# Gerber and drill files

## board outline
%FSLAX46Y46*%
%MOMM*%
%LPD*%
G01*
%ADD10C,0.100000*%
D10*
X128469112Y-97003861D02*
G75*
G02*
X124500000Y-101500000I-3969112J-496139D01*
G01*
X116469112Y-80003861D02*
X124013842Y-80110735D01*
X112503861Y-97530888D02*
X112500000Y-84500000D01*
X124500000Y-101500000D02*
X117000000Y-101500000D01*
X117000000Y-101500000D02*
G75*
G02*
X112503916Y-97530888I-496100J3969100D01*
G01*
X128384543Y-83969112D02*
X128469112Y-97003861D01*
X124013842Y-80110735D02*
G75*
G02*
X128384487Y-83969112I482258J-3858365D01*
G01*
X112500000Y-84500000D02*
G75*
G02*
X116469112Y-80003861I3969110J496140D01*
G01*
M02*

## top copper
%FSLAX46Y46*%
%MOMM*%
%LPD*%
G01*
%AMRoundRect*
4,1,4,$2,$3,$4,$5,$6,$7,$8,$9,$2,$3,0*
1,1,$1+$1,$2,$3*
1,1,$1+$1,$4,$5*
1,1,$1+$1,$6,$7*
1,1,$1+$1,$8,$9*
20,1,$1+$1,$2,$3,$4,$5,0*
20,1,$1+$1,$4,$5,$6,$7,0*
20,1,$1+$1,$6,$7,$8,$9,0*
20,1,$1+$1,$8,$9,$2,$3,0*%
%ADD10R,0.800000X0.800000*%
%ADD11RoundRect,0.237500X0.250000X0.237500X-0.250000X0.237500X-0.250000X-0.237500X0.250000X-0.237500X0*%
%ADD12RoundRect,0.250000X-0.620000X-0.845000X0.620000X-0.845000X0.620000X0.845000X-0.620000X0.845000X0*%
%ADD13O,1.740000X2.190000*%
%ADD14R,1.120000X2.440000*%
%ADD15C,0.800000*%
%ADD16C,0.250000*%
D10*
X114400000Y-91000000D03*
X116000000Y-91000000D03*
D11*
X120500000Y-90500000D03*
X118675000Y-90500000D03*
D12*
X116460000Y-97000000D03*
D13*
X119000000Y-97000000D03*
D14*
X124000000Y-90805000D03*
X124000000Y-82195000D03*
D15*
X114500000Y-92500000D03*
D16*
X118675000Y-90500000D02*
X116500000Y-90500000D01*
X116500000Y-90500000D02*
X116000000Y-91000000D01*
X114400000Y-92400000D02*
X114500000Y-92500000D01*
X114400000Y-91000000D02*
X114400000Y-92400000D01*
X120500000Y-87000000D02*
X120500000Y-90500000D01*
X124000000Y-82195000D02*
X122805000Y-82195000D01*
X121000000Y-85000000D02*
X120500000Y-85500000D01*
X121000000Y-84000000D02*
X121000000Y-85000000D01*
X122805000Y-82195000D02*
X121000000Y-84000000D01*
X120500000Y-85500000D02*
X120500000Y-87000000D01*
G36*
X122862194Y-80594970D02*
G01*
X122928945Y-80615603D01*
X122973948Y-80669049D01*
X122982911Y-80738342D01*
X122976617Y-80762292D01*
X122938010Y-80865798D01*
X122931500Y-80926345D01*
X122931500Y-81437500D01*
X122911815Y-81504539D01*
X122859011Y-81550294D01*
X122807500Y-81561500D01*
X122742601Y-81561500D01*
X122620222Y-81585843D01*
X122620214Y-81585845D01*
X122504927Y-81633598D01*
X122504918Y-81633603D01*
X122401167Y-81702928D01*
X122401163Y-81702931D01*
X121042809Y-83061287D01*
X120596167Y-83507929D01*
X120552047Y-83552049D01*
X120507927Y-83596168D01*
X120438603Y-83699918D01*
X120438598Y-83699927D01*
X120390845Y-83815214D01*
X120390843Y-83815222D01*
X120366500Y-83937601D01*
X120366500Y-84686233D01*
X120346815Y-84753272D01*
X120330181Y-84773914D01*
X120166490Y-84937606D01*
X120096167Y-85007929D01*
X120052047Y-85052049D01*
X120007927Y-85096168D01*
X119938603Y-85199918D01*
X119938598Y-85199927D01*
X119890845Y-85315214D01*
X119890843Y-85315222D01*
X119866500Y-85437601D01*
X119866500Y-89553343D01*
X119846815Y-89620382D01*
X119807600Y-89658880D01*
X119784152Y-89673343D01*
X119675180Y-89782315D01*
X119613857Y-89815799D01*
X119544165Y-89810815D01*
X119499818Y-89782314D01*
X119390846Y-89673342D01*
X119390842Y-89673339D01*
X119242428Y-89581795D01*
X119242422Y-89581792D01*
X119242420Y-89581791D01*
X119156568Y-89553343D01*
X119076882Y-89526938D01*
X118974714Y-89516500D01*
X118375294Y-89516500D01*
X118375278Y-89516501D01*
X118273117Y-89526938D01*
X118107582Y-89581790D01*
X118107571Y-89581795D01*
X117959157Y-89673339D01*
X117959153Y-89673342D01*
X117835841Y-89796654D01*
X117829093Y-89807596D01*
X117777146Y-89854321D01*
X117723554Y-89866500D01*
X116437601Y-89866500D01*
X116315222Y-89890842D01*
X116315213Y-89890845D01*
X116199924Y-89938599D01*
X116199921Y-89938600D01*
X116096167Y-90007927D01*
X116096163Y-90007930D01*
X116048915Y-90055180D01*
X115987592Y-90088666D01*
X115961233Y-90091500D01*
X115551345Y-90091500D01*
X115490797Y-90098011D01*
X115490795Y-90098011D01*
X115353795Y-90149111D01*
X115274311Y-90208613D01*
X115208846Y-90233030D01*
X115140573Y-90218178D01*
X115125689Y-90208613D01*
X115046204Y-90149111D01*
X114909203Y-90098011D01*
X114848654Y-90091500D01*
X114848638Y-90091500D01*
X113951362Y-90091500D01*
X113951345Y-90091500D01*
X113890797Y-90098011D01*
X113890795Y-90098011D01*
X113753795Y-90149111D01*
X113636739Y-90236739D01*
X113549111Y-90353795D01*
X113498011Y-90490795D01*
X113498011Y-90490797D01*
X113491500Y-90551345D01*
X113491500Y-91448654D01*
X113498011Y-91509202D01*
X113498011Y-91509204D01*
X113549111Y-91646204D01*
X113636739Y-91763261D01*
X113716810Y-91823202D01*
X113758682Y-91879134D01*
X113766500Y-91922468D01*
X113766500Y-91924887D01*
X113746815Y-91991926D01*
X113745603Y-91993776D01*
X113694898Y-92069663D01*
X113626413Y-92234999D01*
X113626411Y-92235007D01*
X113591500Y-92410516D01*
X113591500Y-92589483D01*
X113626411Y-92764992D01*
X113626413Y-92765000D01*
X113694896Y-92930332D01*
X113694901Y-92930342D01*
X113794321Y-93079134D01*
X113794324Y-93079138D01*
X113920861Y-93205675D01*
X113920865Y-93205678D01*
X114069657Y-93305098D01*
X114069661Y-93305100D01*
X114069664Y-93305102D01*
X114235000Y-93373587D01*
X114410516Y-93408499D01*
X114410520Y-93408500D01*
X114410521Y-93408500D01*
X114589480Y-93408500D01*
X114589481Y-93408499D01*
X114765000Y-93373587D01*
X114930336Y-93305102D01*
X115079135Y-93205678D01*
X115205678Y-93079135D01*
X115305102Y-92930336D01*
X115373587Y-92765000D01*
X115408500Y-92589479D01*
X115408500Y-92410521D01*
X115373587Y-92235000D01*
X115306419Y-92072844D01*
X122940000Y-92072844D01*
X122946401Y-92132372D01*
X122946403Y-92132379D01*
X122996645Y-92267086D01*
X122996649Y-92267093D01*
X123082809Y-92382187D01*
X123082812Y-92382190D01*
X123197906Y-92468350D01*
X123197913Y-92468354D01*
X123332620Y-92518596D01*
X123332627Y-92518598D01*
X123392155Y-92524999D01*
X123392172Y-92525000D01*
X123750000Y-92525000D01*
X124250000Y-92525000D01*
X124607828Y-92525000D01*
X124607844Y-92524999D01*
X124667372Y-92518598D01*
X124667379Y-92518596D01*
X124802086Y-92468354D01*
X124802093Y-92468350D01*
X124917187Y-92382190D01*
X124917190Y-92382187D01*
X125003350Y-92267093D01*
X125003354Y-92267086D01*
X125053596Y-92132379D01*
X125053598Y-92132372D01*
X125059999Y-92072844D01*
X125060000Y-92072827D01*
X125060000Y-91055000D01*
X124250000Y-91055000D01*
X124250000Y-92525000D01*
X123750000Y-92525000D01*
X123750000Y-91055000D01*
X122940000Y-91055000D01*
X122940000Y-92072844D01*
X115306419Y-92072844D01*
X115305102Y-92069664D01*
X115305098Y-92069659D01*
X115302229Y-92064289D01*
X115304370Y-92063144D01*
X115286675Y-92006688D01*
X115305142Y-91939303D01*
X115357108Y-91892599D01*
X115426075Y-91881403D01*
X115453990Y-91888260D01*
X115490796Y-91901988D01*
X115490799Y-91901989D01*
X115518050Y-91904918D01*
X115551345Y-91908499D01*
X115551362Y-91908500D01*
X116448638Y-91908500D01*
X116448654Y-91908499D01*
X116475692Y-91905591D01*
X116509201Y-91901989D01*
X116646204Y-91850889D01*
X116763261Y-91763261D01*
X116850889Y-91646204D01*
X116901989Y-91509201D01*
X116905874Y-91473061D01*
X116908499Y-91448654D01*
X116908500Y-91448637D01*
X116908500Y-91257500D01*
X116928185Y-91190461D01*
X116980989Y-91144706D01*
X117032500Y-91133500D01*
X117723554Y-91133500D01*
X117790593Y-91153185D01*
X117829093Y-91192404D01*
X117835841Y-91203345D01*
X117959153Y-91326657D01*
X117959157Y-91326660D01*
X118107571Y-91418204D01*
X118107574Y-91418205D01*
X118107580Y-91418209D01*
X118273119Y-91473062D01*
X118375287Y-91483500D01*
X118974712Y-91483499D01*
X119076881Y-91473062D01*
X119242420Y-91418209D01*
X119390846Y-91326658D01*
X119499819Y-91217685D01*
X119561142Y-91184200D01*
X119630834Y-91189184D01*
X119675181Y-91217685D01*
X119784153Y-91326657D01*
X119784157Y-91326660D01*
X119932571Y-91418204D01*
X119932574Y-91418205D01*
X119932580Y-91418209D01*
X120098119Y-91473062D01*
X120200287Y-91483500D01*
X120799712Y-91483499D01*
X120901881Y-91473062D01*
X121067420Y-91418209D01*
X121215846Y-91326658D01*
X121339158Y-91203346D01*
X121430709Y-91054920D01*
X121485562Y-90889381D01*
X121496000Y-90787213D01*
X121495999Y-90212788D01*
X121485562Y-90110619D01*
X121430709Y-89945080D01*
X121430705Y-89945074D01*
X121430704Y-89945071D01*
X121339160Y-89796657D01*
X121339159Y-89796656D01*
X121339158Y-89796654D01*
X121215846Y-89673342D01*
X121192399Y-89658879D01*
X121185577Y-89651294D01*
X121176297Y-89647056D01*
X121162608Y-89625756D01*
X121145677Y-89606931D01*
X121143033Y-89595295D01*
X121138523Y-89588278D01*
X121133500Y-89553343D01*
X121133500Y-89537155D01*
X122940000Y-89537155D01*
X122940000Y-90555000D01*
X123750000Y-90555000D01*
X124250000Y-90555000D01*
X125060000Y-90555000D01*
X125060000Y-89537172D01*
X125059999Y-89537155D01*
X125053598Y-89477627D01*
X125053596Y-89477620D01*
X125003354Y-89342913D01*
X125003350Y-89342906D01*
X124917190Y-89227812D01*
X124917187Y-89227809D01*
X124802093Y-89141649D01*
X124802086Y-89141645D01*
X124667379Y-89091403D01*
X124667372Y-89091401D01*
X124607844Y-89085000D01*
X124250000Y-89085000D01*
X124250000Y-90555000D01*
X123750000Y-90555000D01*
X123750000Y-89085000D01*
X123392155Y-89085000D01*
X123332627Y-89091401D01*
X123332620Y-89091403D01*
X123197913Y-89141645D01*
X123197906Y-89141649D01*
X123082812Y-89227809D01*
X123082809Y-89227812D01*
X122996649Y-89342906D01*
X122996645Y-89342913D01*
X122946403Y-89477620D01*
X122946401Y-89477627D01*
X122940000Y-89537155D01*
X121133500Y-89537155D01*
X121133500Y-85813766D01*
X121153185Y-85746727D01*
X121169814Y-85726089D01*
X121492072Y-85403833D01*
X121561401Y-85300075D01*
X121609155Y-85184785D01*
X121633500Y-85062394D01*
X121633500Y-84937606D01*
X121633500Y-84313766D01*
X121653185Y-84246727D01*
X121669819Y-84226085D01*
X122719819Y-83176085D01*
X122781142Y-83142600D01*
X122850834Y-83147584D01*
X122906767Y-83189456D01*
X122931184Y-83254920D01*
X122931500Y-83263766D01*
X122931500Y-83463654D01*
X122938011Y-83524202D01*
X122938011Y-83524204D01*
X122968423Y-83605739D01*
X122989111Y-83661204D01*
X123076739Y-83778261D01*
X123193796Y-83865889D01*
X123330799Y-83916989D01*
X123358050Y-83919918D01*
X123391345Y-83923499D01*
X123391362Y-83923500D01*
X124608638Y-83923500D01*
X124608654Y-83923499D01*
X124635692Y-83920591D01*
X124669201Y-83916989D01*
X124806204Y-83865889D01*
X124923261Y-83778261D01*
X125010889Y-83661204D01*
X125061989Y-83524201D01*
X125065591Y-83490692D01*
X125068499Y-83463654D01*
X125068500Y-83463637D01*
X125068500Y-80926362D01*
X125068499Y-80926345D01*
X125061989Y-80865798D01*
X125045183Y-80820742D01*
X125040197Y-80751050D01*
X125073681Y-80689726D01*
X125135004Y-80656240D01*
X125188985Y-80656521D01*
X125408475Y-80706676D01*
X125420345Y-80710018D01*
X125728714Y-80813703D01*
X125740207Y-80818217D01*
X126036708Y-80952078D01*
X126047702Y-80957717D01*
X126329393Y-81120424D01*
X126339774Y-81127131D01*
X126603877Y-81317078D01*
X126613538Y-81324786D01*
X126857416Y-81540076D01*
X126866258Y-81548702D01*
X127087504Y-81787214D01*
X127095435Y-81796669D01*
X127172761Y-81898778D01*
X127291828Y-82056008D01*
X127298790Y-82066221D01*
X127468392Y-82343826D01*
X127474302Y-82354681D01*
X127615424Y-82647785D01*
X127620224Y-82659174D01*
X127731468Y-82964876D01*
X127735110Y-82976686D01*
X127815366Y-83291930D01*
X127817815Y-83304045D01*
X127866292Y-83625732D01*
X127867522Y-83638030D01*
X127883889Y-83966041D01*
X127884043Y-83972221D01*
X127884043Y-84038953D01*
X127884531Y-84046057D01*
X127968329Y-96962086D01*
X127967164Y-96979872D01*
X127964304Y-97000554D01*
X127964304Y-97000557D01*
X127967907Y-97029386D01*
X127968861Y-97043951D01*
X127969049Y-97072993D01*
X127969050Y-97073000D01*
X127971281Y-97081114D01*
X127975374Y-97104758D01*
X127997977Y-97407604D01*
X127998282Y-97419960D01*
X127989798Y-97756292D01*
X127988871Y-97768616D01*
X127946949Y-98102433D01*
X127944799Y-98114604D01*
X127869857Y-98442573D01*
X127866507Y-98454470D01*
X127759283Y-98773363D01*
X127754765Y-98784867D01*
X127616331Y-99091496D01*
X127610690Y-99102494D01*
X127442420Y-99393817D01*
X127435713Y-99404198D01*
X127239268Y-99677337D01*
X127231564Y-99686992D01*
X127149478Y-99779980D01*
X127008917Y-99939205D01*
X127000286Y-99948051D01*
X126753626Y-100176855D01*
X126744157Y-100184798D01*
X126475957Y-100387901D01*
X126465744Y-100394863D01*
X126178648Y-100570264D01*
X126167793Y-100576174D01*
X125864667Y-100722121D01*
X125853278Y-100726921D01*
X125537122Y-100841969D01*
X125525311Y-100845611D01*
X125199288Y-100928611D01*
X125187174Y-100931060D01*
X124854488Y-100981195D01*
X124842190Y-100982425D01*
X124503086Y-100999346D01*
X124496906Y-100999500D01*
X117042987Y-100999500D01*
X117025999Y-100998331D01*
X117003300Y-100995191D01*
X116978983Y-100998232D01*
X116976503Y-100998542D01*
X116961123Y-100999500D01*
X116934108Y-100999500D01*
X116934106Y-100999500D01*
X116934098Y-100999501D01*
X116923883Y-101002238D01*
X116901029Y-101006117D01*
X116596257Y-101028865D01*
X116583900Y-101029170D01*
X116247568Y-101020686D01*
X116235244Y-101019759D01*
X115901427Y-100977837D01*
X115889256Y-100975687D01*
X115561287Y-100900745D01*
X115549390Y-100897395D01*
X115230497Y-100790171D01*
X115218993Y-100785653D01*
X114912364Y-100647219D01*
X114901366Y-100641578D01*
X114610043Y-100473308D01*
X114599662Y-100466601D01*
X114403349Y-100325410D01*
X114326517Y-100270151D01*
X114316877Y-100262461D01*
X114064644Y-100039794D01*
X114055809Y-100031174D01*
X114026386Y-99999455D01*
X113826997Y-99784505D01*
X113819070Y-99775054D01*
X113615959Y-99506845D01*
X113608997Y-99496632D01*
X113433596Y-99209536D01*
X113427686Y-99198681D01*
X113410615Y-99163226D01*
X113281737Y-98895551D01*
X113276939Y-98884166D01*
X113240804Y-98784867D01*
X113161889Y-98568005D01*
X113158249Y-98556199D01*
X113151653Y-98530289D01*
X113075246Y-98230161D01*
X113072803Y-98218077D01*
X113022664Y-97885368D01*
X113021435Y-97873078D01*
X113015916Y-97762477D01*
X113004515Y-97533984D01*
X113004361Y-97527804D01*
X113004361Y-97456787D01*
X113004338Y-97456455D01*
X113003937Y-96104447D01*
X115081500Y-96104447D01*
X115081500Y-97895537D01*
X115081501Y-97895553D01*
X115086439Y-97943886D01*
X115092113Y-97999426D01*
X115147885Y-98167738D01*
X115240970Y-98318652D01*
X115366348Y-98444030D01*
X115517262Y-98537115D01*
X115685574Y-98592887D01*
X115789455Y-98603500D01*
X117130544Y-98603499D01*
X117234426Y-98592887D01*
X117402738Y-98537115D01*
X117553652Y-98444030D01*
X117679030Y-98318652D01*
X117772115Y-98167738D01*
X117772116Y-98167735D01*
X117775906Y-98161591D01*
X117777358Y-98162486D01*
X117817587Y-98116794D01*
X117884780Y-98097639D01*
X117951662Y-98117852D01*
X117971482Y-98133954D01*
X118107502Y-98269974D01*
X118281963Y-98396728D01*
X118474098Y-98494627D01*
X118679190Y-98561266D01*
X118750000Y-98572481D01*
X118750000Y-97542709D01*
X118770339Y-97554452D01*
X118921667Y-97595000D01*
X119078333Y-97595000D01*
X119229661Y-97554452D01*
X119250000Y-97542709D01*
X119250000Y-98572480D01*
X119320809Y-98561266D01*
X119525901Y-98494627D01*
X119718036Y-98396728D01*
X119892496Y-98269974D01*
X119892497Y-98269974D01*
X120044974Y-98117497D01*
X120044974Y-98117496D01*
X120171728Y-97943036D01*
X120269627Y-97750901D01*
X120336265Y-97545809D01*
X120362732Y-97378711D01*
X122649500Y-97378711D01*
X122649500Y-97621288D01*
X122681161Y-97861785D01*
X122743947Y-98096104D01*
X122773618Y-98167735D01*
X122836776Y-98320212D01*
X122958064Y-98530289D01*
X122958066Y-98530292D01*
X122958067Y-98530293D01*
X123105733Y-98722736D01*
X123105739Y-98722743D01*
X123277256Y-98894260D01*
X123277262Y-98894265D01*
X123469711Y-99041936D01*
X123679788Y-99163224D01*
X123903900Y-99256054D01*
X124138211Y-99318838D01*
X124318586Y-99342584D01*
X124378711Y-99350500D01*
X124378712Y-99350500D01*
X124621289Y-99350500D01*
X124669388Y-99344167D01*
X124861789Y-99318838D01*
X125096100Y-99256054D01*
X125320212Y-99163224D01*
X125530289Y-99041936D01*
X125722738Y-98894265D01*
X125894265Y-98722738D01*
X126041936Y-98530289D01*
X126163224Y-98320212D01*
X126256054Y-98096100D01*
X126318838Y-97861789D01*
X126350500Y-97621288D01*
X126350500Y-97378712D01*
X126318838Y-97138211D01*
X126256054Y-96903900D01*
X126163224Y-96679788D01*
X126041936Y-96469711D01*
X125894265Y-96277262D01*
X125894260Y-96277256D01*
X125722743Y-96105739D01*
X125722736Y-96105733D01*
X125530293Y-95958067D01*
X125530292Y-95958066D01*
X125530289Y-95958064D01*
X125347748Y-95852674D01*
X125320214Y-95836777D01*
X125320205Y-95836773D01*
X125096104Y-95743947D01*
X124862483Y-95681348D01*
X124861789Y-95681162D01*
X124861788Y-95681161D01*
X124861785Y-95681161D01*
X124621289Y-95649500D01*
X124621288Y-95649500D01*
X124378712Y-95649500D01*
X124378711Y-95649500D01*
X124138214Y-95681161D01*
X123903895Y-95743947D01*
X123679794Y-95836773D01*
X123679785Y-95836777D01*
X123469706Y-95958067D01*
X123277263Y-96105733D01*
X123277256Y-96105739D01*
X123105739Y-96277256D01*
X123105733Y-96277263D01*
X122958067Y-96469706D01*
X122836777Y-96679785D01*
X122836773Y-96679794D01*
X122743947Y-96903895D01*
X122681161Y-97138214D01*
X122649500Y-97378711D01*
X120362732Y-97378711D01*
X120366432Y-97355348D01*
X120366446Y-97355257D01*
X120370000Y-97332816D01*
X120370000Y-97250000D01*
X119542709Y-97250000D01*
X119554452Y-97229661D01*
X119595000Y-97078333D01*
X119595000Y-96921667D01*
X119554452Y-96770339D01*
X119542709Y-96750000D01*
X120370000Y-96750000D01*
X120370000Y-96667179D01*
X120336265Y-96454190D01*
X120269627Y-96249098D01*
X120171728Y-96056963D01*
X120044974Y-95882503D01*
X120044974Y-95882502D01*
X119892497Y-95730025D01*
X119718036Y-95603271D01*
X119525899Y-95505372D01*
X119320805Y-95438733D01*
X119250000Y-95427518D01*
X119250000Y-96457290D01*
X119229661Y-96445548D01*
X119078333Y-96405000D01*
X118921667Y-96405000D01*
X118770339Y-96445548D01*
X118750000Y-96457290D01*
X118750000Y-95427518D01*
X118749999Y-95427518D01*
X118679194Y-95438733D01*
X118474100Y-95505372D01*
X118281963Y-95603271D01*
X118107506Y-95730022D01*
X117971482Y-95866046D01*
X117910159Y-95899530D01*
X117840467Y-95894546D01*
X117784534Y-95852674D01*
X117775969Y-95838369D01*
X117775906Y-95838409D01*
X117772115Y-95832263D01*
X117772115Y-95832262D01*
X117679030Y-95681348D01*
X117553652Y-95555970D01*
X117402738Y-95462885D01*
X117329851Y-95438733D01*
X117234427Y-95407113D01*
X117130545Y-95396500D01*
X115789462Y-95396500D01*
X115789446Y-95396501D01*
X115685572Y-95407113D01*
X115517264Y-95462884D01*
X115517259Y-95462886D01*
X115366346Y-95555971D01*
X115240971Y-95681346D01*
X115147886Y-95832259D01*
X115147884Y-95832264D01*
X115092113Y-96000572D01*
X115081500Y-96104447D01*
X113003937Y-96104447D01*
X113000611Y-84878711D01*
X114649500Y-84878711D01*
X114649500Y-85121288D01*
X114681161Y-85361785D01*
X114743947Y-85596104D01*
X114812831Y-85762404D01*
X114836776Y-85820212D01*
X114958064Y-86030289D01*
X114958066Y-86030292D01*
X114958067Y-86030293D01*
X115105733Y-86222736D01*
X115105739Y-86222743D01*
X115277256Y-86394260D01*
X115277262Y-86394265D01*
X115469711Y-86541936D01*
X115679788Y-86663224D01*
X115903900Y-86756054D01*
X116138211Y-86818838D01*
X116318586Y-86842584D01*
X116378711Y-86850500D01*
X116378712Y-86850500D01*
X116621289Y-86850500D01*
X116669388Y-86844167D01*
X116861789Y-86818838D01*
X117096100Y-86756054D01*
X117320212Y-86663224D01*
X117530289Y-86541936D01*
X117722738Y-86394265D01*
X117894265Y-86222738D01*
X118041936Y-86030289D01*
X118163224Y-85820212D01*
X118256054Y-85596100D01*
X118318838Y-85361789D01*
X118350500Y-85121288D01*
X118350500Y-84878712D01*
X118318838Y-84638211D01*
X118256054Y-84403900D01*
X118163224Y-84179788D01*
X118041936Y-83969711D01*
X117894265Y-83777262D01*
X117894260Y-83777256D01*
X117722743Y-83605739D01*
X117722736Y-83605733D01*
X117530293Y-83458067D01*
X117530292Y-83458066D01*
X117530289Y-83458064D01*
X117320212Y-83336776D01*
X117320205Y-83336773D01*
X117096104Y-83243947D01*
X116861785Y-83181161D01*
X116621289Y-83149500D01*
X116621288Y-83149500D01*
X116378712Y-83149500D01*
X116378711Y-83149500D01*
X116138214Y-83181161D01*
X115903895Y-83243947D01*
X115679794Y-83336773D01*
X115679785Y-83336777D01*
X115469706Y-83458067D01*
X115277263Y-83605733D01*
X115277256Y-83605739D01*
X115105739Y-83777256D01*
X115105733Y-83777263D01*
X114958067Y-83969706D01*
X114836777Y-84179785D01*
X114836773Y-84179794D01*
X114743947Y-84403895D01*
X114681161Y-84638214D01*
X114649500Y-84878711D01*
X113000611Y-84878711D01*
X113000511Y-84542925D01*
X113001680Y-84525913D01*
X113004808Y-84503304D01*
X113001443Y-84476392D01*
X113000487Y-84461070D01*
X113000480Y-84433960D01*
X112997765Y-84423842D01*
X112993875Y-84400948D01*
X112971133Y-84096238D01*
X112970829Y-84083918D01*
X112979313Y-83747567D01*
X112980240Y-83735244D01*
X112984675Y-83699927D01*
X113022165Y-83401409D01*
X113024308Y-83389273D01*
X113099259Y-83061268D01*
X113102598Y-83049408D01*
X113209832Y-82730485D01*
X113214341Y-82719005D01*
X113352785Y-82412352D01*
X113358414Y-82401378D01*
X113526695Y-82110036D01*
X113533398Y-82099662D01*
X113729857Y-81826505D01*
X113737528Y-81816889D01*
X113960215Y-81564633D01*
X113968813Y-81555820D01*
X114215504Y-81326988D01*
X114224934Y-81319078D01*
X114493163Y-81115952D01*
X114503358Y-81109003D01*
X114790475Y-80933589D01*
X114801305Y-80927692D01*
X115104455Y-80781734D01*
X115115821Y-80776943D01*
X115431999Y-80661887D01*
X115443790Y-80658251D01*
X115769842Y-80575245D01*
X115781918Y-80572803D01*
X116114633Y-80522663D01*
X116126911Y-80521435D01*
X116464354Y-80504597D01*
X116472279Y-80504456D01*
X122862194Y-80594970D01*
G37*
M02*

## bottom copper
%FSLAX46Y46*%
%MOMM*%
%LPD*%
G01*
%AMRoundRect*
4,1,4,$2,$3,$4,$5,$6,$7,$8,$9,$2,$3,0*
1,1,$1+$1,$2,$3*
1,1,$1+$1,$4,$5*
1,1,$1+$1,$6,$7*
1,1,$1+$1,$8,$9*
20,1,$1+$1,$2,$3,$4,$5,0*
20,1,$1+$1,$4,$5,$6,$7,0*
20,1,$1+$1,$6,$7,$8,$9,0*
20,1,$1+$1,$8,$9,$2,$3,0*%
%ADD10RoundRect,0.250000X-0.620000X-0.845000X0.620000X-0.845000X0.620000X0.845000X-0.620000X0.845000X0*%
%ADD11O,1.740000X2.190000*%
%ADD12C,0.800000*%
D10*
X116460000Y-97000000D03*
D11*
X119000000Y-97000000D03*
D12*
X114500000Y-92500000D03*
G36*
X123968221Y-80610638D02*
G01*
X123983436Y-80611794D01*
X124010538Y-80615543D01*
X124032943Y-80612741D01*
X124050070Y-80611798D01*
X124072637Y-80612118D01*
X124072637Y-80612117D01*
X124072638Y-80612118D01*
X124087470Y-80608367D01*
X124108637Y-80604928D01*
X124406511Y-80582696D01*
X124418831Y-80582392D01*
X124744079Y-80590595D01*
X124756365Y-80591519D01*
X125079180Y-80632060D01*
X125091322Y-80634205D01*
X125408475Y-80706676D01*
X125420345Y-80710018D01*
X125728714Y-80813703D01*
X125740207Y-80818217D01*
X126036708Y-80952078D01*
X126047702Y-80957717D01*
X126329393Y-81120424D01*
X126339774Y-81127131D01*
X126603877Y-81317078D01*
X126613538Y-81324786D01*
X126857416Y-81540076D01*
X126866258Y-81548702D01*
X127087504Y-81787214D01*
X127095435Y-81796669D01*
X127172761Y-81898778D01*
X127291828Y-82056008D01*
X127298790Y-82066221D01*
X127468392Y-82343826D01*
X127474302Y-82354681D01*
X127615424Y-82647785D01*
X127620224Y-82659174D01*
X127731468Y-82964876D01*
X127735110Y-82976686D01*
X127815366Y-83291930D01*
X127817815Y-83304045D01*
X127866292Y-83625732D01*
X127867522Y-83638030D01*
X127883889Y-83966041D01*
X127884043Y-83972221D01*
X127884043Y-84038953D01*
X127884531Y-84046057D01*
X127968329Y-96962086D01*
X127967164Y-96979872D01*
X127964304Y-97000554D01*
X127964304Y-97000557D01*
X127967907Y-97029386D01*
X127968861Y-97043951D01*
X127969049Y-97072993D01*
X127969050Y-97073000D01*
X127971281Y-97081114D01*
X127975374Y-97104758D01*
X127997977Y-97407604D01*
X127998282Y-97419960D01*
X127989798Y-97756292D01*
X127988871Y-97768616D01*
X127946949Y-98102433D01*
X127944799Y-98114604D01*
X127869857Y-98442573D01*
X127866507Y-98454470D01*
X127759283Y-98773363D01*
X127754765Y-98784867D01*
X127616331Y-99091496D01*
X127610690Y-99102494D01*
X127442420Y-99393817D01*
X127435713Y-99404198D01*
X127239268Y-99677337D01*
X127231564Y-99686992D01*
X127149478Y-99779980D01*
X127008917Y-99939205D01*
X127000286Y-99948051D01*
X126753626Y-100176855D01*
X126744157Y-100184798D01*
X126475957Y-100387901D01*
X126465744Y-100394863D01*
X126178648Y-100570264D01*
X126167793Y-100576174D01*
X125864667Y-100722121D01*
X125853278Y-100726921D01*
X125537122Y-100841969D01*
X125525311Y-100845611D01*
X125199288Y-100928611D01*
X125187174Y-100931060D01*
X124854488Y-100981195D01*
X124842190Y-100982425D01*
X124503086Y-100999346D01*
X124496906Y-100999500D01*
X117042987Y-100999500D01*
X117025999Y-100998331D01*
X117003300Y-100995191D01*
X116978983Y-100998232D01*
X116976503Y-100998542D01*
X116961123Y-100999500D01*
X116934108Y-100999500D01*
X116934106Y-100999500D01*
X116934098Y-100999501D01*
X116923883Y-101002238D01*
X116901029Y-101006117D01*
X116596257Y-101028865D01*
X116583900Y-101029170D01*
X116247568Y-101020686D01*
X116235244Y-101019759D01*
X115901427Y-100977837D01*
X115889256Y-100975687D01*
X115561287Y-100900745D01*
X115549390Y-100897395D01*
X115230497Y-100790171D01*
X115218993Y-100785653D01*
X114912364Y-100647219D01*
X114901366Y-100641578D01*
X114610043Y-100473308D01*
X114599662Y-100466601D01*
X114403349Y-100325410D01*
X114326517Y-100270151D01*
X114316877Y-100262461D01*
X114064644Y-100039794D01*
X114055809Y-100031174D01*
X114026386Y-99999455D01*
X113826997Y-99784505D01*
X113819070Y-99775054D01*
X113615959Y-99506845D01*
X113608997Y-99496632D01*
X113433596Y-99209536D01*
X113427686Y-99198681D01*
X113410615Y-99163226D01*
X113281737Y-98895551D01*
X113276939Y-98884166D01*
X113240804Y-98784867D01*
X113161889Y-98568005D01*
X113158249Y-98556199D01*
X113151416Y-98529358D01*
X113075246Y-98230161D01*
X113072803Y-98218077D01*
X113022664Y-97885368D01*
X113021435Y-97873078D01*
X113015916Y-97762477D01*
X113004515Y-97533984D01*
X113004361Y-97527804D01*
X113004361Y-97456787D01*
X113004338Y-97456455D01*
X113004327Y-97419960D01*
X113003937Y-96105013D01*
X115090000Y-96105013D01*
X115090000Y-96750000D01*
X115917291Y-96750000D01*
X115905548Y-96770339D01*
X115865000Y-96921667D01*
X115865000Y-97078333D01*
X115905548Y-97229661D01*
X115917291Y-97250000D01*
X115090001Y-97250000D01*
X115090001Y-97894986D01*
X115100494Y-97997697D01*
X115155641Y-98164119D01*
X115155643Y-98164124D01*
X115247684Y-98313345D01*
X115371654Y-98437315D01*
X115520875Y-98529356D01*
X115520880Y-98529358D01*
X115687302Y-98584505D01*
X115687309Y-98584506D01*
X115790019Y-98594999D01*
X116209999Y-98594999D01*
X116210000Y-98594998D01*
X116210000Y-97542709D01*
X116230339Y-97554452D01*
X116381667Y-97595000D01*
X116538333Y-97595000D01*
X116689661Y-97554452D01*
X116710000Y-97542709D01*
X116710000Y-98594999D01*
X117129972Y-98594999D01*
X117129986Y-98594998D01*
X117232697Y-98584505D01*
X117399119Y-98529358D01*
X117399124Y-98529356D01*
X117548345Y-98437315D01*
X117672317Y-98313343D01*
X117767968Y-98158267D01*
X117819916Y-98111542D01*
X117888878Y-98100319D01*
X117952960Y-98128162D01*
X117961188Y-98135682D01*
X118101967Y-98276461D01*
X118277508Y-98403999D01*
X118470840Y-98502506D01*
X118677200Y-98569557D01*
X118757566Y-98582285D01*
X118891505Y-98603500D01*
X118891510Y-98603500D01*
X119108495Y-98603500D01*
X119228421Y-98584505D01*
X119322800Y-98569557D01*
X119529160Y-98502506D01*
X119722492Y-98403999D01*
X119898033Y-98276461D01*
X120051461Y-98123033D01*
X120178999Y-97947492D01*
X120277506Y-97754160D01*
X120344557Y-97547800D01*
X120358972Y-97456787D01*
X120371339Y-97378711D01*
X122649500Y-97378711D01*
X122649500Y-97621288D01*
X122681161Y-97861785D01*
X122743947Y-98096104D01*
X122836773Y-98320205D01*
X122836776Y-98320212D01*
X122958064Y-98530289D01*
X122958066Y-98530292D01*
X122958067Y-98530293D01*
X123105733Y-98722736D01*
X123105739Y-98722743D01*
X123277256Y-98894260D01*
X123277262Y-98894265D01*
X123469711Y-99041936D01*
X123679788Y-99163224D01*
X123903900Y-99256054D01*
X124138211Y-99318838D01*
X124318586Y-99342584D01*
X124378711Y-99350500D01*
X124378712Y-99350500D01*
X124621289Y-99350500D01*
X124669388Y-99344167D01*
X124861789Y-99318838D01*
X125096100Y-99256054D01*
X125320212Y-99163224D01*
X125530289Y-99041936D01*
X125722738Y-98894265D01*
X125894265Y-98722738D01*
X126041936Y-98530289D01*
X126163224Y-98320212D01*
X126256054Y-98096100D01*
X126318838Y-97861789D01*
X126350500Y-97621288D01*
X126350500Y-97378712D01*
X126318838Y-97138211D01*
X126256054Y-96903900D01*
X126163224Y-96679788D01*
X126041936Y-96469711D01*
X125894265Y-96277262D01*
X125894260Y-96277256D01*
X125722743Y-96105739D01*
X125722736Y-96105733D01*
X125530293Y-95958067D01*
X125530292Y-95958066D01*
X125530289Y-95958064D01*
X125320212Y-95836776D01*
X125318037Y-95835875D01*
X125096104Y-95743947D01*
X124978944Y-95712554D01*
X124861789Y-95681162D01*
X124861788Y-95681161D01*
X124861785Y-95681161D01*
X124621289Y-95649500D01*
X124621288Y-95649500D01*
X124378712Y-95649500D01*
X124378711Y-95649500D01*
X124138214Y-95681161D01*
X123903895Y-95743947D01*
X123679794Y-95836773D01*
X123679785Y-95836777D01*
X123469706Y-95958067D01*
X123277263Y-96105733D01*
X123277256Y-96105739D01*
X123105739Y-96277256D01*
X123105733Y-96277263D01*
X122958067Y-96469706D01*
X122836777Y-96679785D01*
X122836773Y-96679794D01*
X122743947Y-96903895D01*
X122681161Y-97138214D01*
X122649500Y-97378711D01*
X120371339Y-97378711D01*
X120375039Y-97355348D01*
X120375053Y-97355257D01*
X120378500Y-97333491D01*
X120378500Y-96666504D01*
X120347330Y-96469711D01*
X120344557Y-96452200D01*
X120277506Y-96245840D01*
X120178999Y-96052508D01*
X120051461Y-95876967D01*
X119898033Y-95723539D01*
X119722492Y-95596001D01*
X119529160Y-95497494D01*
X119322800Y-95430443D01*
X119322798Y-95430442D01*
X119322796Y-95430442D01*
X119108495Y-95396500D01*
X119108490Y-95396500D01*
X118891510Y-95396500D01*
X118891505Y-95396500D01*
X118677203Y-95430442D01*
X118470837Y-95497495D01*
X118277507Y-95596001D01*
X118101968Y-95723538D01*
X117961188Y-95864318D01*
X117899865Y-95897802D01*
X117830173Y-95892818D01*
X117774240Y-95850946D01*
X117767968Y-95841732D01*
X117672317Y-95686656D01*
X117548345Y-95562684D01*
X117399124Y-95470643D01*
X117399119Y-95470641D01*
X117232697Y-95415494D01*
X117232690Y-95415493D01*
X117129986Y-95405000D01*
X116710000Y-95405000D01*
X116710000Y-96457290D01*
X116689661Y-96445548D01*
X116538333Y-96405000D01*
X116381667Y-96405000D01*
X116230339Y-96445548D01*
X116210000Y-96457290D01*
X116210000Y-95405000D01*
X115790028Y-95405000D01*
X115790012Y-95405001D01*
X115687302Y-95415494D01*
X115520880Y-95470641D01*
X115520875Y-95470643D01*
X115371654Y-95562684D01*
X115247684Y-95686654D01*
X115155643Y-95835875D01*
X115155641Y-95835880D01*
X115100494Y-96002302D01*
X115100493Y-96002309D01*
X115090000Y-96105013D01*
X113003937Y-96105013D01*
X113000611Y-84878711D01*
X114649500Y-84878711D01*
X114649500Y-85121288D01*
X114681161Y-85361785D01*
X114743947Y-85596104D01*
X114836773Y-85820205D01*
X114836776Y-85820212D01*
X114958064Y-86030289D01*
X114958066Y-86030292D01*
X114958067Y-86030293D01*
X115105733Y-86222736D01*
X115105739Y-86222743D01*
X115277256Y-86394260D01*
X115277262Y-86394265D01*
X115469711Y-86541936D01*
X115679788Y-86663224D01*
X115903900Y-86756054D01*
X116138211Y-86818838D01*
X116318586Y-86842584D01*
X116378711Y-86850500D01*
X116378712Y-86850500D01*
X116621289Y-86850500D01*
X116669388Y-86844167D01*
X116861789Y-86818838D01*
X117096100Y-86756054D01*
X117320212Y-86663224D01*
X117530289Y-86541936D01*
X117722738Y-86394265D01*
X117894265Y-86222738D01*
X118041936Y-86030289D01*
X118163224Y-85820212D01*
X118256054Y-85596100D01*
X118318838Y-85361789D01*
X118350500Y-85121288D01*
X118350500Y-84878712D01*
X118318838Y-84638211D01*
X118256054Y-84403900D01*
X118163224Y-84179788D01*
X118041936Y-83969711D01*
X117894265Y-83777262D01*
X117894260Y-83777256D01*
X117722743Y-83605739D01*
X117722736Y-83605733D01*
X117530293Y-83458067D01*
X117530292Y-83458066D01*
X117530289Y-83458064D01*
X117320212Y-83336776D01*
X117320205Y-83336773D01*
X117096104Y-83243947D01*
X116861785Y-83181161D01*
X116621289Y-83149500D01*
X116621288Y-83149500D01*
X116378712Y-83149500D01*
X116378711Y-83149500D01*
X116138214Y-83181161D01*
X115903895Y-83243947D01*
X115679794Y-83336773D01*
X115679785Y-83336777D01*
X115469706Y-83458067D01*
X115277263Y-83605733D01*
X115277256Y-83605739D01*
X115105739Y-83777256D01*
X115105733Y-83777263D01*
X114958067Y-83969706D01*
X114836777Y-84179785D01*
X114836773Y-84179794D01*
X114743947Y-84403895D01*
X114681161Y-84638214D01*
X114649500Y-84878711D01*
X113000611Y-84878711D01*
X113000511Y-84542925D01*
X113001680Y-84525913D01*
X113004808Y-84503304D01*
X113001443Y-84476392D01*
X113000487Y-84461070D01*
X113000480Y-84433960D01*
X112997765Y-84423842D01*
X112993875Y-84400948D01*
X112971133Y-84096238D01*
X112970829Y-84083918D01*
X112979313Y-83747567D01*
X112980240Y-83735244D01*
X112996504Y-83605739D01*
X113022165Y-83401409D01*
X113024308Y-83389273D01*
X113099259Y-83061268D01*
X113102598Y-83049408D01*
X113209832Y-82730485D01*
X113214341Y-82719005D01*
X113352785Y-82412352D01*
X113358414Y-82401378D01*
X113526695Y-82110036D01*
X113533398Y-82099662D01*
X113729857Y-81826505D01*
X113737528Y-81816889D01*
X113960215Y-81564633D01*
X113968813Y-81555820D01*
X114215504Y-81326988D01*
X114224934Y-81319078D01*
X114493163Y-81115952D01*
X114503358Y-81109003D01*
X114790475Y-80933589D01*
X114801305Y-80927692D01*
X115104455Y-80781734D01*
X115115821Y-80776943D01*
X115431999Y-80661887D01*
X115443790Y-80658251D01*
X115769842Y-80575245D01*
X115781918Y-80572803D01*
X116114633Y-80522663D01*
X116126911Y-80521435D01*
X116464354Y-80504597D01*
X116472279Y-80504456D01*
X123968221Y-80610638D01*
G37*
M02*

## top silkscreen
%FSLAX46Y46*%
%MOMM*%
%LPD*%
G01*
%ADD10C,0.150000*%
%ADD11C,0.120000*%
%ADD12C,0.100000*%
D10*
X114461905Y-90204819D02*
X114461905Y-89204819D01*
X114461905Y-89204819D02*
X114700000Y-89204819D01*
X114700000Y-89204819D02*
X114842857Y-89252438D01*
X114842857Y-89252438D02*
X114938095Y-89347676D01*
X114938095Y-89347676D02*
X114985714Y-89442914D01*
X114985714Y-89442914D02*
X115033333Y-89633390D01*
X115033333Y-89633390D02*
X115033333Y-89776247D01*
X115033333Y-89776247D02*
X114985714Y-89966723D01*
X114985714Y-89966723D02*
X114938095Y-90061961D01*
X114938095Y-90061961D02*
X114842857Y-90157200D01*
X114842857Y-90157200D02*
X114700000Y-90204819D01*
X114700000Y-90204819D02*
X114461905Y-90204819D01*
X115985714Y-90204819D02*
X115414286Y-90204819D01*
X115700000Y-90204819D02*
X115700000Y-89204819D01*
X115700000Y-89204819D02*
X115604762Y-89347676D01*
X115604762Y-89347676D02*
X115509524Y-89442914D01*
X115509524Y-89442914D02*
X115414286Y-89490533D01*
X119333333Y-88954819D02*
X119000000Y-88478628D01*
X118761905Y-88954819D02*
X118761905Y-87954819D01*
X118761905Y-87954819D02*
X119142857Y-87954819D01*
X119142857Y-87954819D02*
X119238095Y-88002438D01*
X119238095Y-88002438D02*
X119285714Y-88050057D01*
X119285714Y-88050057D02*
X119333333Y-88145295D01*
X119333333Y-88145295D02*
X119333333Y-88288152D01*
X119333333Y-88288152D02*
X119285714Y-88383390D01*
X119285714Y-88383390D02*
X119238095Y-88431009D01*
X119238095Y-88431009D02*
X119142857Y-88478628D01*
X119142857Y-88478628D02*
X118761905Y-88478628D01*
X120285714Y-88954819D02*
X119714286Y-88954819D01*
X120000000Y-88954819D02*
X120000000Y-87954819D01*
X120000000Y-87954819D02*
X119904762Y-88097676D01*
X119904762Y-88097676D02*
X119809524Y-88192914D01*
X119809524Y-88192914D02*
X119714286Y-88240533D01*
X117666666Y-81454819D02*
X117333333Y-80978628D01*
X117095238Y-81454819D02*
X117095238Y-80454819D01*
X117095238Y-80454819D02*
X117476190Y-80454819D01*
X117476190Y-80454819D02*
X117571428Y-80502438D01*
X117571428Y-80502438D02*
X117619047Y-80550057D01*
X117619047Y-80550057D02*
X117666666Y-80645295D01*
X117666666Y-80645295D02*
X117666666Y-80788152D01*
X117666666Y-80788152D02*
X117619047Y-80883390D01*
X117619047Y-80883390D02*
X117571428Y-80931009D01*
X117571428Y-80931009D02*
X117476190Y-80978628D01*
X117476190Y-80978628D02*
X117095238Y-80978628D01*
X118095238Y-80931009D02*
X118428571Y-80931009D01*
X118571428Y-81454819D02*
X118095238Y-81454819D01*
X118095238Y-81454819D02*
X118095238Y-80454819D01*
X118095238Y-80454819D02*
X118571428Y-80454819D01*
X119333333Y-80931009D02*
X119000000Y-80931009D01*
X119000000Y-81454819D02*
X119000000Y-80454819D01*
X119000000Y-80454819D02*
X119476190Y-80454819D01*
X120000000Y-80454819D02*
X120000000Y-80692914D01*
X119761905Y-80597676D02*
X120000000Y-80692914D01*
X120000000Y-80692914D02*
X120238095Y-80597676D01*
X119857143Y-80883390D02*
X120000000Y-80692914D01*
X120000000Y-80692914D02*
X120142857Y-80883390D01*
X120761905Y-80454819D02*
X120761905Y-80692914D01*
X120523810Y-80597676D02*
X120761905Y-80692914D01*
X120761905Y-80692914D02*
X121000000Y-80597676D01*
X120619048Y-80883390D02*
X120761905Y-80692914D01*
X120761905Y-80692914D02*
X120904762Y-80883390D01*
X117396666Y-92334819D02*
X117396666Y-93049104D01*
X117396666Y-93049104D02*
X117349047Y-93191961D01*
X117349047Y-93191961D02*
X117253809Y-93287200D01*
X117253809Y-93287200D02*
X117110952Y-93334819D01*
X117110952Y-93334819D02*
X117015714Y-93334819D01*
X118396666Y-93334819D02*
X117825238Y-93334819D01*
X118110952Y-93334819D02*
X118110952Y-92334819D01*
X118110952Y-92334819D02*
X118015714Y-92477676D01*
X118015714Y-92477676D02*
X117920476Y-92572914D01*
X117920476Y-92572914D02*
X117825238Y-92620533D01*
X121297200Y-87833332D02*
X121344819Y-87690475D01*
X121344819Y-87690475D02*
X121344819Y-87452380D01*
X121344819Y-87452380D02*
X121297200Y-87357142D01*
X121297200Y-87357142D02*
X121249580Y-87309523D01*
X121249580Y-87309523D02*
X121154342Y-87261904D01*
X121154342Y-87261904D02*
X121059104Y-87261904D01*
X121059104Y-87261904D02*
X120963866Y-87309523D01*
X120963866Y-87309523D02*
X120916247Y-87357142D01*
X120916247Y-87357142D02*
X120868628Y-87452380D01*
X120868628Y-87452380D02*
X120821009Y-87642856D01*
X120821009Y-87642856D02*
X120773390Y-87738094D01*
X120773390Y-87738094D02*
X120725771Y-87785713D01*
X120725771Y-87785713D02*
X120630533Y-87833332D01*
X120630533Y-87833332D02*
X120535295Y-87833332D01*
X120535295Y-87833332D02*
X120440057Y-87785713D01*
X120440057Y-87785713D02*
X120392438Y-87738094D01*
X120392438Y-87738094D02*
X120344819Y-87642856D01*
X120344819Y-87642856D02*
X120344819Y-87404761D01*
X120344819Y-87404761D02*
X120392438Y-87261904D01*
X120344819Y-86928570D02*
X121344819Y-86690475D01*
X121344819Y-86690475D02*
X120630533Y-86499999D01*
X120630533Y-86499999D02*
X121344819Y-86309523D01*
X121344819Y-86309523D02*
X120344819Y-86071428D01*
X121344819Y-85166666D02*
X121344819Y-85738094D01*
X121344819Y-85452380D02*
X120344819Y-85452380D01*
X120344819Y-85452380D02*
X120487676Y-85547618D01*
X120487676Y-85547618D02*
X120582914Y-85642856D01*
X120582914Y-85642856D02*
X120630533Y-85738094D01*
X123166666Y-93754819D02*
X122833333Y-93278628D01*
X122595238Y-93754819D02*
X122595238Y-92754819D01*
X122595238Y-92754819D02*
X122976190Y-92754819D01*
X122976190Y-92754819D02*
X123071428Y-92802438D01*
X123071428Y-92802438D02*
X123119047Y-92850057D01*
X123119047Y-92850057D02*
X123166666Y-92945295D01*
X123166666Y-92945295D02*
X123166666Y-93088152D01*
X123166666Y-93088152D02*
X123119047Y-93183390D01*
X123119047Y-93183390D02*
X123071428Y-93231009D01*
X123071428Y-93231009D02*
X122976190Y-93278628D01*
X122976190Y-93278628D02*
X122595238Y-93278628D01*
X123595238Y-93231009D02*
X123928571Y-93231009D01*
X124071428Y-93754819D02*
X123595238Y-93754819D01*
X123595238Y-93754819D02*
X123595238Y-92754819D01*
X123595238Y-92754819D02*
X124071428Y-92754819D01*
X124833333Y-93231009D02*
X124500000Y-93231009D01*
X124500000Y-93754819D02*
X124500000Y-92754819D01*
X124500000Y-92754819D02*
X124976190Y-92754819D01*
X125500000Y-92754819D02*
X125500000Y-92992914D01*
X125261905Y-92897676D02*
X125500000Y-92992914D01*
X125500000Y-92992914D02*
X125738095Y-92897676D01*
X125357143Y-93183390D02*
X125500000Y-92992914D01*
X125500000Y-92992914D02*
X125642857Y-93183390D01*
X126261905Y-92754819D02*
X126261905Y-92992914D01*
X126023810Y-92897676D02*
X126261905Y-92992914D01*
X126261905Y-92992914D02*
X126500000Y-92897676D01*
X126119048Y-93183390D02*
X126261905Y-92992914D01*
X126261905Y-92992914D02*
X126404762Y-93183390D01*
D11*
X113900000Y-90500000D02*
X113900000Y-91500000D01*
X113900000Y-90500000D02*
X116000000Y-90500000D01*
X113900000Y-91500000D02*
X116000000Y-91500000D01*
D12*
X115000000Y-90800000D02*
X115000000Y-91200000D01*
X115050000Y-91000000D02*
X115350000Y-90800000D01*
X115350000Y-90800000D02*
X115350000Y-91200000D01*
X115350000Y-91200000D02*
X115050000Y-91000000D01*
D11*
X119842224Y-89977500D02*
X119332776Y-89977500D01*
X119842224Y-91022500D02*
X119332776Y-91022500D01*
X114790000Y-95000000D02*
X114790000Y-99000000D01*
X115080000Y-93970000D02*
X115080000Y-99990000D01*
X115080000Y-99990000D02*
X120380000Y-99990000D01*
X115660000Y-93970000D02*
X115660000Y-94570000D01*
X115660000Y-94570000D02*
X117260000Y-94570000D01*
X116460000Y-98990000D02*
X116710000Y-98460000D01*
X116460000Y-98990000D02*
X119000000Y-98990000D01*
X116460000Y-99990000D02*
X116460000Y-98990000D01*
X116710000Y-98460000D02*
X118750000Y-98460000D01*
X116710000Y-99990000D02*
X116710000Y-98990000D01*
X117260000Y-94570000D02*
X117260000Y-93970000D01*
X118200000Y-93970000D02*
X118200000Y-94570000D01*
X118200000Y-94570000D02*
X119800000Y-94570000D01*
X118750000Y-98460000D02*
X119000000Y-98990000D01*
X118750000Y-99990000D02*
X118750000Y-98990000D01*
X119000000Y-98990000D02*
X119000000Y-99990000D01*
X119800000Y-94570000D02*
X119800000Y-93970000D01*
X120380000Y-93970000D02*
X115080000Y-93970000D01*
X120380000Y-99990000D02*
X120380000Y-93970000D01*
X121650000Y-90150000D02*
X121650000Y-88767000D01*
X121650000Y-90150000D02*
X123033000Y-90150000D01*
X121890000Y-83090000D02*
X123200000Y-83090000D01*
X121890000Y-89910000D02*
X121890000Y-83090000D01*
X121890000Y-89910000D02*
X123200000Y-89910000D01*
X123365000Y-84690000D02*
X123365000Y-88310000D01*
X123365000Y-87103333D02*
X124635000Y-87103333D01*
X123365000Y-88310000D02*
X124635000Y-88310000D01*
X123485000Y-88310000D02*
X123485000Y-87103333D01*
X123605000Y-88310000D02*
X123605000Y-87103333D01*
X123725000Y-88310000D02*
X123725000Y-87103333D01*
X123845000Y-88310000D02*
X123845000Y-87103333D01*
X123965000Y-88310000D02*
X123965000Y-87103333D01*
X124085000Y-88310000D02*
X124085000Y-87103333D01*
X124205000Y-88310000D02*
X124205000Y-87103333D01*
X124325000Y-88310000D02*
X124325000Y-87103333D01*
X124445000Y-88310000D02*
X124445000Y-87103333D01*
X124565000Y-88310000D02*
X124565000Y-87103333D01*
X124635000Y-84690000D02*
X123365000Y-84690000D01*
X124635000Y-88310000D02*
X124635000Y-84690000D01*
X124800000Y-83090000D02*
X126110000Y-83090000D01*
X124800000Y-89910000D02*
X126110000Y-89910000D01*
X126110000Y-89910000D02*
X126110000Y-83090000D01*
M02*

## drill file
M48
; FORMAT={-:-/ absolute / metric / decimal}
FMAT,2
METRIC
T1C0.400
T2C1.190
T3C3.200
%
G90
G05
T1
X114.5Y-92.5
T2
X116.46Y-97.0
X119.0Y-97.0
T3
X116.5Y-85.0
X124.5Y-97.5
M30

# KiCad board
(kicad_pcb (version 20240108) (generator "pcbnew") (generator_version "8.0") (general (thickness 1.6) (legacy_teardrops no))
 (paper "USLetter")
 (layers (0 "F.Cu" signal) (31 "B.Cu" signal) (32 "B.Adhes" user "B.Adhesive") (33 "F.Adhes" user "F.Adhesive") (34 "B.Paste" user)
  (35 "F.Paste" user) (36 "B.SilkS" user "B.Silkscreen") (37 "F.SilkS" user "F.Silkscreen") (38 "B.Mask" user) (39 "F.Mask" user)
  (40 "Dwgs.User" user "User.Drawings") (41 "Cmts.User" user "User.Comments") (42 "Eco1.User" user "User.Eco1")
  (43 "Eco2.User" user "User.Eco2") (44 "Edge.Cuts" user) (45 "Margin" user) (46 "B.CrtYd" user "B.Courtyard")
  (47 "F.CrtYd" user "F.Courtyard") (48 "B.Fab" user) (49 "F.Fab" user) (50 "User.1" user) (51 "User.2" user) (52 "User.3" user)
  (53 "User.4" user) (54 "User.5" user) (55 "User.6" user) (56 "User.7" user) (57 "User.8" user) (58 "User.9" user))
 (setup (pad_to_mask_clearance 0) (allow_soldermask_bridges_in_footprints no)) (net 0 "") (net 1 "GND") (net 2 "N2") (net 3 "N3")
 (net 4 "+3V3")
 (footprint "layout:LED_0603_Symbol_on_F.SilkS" (layer "F.Cu") (at 115.2 91)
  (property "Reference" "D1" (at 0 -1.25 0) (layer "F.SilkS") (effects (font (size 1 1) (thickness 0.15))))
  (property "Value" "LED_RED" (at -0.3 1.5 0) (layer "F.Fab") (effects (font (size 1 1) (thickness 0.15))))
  (fp_line (start -1.3 -0.5) (end -1.3 0.5) (stroke (width 0.12) (type solid)) (layer "F.SilkS"))
  (fp_line (start -1.3 -0.5) (end 0.8 -0.5) (stroke (width 0.12) (type solid)) (layer "F.SilkS"))
  (fp_line (start -1.3 0.5) (end 0.8 0.5) (stroke (width 0.12) (type solid)) (layer "F.SilkS"))
  (fp_line (start -0.2 -0.2) (end -0.2 0.2) (stroke (width 0.1) (type solid)) (layer "F.SilkS"))
  (fp_line (start -0.15 0) (end 0.15 -0.2) (stroke (width 0.1) (type solid)) (layer "F.SilkS"))
  (fp_line (start 0.15 -0.2) (end 0.15 0.2) (stroke (width 0.1) (type solid)) (layer "F.SilkS"))
  (fp_line (start 0.15 0.2) (end -0.15 0) (stroke (width 0.1) (type solid)) (layer "F.SilkS"))
  (pad "1" smd rect (at -0.8 0 180) (size 0.8 0.8) (layers "F.Cu" "F.Paste" "F.Mask") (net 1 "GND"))
  (pad "2" smd rect (at 0.8 0 180) (size 0.8 0.8) (layers "F.Cu" "F.Paste" "F.Mask") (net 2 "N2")))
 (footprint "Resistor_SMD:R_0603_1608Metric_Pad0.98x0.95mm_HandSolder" (layer "F.Cu") (at 119.5875 90.5 180)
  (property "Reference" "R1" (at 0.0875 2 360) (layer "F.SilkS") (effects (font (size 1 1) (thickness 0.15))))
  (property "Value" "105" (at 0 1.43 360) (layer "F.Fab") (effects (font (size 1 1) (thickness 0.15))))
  (fp_line (start -0.254724 0.5225) (end 0.254724 0.5225) (stroke (width 0.12) (type solid)) (layer "F.SilkS"))
  (fp_line (start -0.254724 -0.5225) (end 0.254724 -0.5225) (stroke (width 0.12) (type solid)) (layer "F.SilkS"))
  (pad "1" smd roundrect (at -0.9125 0 180) (size 0.975 0.95) (layers "F.Cu" "F.Paste" "F.Mask") (roundrect_rratio 0.25) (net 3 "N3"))
  (pad "2" smd roundrect (at 0.9125 0 180) (size 0.975 0.95) (layers "F.Cu" "F.Paste" "F.Mask") (roundrect_rratio 0.25) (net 2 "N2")))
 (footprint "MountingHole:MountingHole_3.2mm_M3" (layer "F.Cu") (at 116.5 85)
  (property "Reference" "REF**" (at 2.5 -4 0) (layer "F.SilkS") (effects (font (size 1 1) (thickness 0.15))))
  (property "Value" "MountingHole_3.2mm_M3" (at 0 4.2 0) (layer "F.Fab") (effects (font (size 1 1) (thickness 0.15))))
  (pad "" np_thru_hole circle (at 0 0) (size 3.2 3.2) (drill 3.2) (layers "*.Cu" "*.Mask")))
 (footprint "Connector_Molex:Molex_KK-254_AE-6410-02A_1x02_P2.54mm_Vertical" (layer "F.Cu") (at 116.46 97)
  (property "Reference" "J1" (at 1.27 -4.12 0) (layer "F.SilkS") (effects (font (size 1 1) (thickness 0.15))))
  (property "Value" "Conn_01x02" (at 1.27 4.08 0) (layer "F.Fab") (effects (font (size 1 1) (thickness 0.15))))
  (fp_line (start -1.67 -2) (end -1.67 2) (stroke (width 0.12) (type solid)) (layer "F.SilkS"))
  (fp_line (start -1.38 -3.03) (end -1.38 2.99) (stroke (width 0.12) (type solid)) (layer "F.SilkS"))
  (fp_line (start -1.38 2.99) (end 3.92 2.99) (stroke (width 0.12) (type solid)) (layer "F.SilkS"))
  (fp_line (start -0.8 -3.03) (end -0.8 -2.43) (stroke (width 0.12) (type solid)) (layer "F.SilkS"))
  (fp_line (start -0.8 -2.43) (end 0.8 -2.43) (stroke (width 0.12) (type solid)) (layer "F.SilkS"))
  (fp_line (start 0 1.99) (end 0.25 1.46) (stroke (width 0.12) (type solid)) (layer "F.SilkS"))
  (fp_line (start 0 1.99) (end 2.54 1.99) (stroke (width 0.12) (type solid)) (layer "F.SilkS"))
  (fp_line (start 0 2.99) (end 0 1.99) (stroke (width 0.12) (type solid)) (layer "F.SilkS"))
  (fp_line (start 0.25 1.46) (end 2.29 1.46) (stroke (width 0.12) (type solid)) (layer "F.SilkS"))
  (fp_line (start 0.25 2.99) (end 0.25 1.99) (stroke (width 0.12) (type solid)) (layer "F.SilkS"))
  (fp_line (start 0.8 -2.43) (end 0.8 -3.03) (stroke (width 0.12) (type solid)) (layer "F.SilkS"))
  (fp_line (start 1.74 -3.03) (end 1.74 -2.43) (stroke (width 0.12) (type solid)) (layer "F.SilkS"))
  (fp_line (start 1.74 -2.43) (end 3.34 -2.43) (stroke (width 0.12) (type solid)) (layer "F.SilkS"))
  (fp_line (start 2.29 1.46) (end 2.54 1.99) (stroke (width 0.12) (type solid)) (layer "F.SilkS"))
  (fp_line (start 2.29 2.99) (end 2.29 1.99) (stroke (width 0.12) (type solid)) (layer "F.SilkS"))
  (fp_line (start 2.54 1.99) (end 2.54 2.99) (stroke (width 0.12) (type solid)) (layer "F.SilkS"))
  (fp_line (start 3.34 -2.43) (end 3.34 -3.03) (stroke (width 0.12) (type solid)) (layer "F.SilkS"))
  (fp_line (start 3.92 -3.03) (end -1.38 -3.03) (stroke (width 0.12) (type solid)) (layer "F.SilkS"))
  (fp_line (start 3.92 2.99) (end 3.92 -3.03) (stroke (width 0.12) (type solid)) (layer "F.SilkS"))
  (pad "1" thru_hole roundrect (at 0 0) (size 1.74 2.19) (drill 1.19) (layers "*.Cu" "*.Mask") (remove_unused_layers no)
   (roundrect_rratio 0.143678) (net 1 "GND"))
  (pad "2" thru_hole oval (at 2.54 0) (size 1.74 2.19) (drill 1.19) (layers "*.Cu" "*.Mask") (remove_unused_layers no) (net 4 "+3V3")))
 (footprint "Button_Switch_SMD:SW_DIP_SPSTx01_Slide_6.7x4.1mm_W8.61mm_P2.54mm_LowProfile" (layer "F.Cu") (at 124 86.5 90)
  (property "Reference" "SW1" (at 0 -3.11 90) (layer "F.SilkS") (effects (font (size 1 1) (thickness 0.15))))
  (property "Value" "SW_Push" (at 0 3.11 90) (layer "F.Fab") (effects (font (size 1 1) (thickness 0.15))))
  (fp_line (start -3.65 -2.35) (end -2.267 -2.35) (stroke (width 0.12) (type solid)) (layer "F.SilkS"))
  (fp_line (start -3.65 -2.35) (end -3.65 -0.967) (stroke (width 0.12) (type solid)) (layer "F.SilkS"))
  (fp_line (start 3.41 -2.11) (end 3.41 -0.8) (stroke (width 0.12) (type solid)) (layer "F.SilkS"))
  (fp_line (start -3.41 -2.11) (end 3.41 -2.11) (stroke (width 0.12) (type solid)) (layer "F.SilkS"))
  (fp_line (start -3.41 -2.11) (end -3.41 -0.8) (stroke (width 0.12) (type solid)) (layer "F.SilkS"))
  (fp_line (start 1.81 -0.635) (end -1.81 -0.635) (stroke (width 0.12) (type solid)) (layer "F.SilkS"))
  (fp_line (start -0.603333 -0.635) (end -0.603333 0.635) (stroke (width 0.12) (type solid)) (layer "F.SilkS"))
  (fp_line (start -1.81 -0.635) (end -1.81 0.635) (stroke (width 0.12) (type solid)) (layer "F.SilkS"))
  (fp_line (start -1.81 -0.515) (end -0.603333 -0.515) (stroke (width 0.12) (type solid)) (layer "F.SilkS"))
  (fp_line (start -1.81 -0.395) (end -0.603333 -0.395) (stroke (width 0.12) (type solid)) (layer "F.SilkS"))
  (fp_line (start -1.81 -0.275) (end -0.603333 -0.275) (stroke (width 0.12) (type solid)) (layer "F.SilkS"))
  (fp_line (start -1.81 -0.155) (end -0.603333 -0.155) (stroke (width 0.12) (type solid)) (layer "F.SilkS"))
  (fp_line (start -1.81 -0.035) (end -0.603333 -0.035) (stroke (width 0.12) (type solid)) (layer "F.SilkS"))
  (fp_line (start -1.81 0.085) (end -0.603333 0.085) (stroke (width 0.12) (type solid)) (layer "F.SilkS"))
  (fp_line (start -1.81 0.205) (end -0.603333 0.205) (stroke (width 0.12) (type solid)) (layer "F.SilkS"))
  (fp_line (start -1.81 0.325) (end -0.603333 0.325) (stroke (width 0.12) (type solid)) (layer "F.SilkS"))
  (fp_line (start -1.81 0.445) (end -0.603333 0.445) (stroke (width 0.12) (type solid)) (layer "F.SilkS"))
  (fp_line (start -1.81 0.565) (end -0.603333 0.565) (stroke (width 0.12) (type solid)) (layer "F.SilkS"))
  (fp_line (start 1.81 0.635) (end 1.81 -0.635) (stroke (width 0.12) (type solid)) (layer "F.SilkS"))
  (fp_line (start -1.81 0.635) (end 1.81 0.635) (stroke (width 0.12) (type solid)) (layer "F.SilkS"))
  (fp_line (start 3.41 0.8) (end 3.41 2.11) (stroke (width 0.12) (type solid)) (layer "F.SilkS"))
  (fp_line (start -3.41 0.8) (end -3.41 2.11) (stroke (width 0.12) (type solid)) (layer "F.SilkS"))
  (fp_line (start -3.41 2.11) (end 3.41 2.11) (stroke (width 0.12) (type solid)) (layer "F.SilkS"))
  (pad "1" smd rect (at -4.305 0 90) (size 2.44 1.12) (layers "F.Cu" "F.Paste" "F.Mask") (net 4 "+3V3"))
  (pad "2" smd rect (at 4.305 0 90) (size 2.44 1.12) (layers "F.Cu" "F.Paste" "F.Mask") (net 3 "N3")))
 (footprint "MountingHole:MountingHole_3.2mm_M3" (layer "F.Cu") (at 124.5 97.5)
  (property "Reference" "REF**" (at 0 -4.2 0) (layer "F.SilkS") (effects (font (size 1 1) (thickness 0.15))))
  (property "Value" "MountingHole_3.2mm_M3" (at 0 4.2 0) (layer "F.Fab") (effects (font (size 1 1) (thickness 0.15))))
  (pad "" np_thru_hole circle (at 0 0) (size 3.2 3.2) (drill 3.2) (layers "*.Cu" "*.Mask")))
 (gr_arc (start 128.469112 97.003861) (mid 127.498713 100.147211) (end 124.5 101.5) (stroke (width 0.1) (type default)) (layer "Edge.Cuts"))
 (gr_line (start 116.469112 80.003861) (end 124.013842 80.110735) (stroke (width 0.1) (type default)) (layer "Edge.Cuts"))
 (gr_line (start 112.503861 97.530888) (end 112.5 84.5) (stroke (width 0.1) (type default)) (layer "Edge.Cuts"))
 (gr_line (start 124.5 101.5) (end 117 101.5) (stroke (width 0.1) (type default)) (layer "Edge.Cuts"))
 (gr_arc (start 117 101.5) (mid 113.85665 100.529601) (end 112.503861 97.530888) (stroke (width 0.1) (type default)) (layer "Edge.Cuts"))
 (gr_line (start 128.384543 83.969112) (end 128.469112 97.003861) (stroke (width 0.1) (type default)) (layer "Edge.Cuts"))
 (gr_arc (start 124.013842 80.110735) (mid 127.069495 81.05406) (end 128.384543 83.969112) (stroke (width 0.1) (type default))
  (layer "Edge.Cuts"))
 (gr_arc (start 112.5 84.5) (mid 113.470399 81.35665) (end 116.469112 80.003861) (stroke (width 0.1) (type default)) (layer "Edge.Cuts"))
 (segment (start 118.675 90.5) (end 116.5 90.5) (width 0.25) (layer "F.Cu") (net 2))
 (segment (start 116.5 90.5) (end 116 91) (width 0.25) (layer "F.Cu") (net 2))
 (segment (start 114.4 92.4) (end 114.5 92.5) (width 0.25) (layer "F.Cu") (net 1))
 (segment (start 114.4 91) (end 114.4 92.4) (width 0.25) (layer "F.Cu") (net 1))
 (via (at 114.5 92.5) (size 0.8) (drill 0.4) (layers "F.Cu" "B.Cu") (free yes) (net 1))
 (segment (start 120.5 87) (end 120.5 90.5) (width 0.25) (layer "F.Cu") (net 3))
 (segment (start 124 82.195) (end 122.805 82.195) (width 0.25) (layer "F.Cu") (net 3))
 (segment (start 121 85) (end 120.5 85.5) (width 0.25) (layer "F.Cu") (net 3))
 (segment (start 121 84) (end 121 85) (width 0.25) (layer "F.Cu") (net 3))
 (segment (start 122.805 82.195) (end 121 84) (width 0.25) (layer "F.Cu") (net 3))
 (segment (start 120.5 85.5) (end 120.5 87) (width 0.25) (layer "F.Cu") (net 3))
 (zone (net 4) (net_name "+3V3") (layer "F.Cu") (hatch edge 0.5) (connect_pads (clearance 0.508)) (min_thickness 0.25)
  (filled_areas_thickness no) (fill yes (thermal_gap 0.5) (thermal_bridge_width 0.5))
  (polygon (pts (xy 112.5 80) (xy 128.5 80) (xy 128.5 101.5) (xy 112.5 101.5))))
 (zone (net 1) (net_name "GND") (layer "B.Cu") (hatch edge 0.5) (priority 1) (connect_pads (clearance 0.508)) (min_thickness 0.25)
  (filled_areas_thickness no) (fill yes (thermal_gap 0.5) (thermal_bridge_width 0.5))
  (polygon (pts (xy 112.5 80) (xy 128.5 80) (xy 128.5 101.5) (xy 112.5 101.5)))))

